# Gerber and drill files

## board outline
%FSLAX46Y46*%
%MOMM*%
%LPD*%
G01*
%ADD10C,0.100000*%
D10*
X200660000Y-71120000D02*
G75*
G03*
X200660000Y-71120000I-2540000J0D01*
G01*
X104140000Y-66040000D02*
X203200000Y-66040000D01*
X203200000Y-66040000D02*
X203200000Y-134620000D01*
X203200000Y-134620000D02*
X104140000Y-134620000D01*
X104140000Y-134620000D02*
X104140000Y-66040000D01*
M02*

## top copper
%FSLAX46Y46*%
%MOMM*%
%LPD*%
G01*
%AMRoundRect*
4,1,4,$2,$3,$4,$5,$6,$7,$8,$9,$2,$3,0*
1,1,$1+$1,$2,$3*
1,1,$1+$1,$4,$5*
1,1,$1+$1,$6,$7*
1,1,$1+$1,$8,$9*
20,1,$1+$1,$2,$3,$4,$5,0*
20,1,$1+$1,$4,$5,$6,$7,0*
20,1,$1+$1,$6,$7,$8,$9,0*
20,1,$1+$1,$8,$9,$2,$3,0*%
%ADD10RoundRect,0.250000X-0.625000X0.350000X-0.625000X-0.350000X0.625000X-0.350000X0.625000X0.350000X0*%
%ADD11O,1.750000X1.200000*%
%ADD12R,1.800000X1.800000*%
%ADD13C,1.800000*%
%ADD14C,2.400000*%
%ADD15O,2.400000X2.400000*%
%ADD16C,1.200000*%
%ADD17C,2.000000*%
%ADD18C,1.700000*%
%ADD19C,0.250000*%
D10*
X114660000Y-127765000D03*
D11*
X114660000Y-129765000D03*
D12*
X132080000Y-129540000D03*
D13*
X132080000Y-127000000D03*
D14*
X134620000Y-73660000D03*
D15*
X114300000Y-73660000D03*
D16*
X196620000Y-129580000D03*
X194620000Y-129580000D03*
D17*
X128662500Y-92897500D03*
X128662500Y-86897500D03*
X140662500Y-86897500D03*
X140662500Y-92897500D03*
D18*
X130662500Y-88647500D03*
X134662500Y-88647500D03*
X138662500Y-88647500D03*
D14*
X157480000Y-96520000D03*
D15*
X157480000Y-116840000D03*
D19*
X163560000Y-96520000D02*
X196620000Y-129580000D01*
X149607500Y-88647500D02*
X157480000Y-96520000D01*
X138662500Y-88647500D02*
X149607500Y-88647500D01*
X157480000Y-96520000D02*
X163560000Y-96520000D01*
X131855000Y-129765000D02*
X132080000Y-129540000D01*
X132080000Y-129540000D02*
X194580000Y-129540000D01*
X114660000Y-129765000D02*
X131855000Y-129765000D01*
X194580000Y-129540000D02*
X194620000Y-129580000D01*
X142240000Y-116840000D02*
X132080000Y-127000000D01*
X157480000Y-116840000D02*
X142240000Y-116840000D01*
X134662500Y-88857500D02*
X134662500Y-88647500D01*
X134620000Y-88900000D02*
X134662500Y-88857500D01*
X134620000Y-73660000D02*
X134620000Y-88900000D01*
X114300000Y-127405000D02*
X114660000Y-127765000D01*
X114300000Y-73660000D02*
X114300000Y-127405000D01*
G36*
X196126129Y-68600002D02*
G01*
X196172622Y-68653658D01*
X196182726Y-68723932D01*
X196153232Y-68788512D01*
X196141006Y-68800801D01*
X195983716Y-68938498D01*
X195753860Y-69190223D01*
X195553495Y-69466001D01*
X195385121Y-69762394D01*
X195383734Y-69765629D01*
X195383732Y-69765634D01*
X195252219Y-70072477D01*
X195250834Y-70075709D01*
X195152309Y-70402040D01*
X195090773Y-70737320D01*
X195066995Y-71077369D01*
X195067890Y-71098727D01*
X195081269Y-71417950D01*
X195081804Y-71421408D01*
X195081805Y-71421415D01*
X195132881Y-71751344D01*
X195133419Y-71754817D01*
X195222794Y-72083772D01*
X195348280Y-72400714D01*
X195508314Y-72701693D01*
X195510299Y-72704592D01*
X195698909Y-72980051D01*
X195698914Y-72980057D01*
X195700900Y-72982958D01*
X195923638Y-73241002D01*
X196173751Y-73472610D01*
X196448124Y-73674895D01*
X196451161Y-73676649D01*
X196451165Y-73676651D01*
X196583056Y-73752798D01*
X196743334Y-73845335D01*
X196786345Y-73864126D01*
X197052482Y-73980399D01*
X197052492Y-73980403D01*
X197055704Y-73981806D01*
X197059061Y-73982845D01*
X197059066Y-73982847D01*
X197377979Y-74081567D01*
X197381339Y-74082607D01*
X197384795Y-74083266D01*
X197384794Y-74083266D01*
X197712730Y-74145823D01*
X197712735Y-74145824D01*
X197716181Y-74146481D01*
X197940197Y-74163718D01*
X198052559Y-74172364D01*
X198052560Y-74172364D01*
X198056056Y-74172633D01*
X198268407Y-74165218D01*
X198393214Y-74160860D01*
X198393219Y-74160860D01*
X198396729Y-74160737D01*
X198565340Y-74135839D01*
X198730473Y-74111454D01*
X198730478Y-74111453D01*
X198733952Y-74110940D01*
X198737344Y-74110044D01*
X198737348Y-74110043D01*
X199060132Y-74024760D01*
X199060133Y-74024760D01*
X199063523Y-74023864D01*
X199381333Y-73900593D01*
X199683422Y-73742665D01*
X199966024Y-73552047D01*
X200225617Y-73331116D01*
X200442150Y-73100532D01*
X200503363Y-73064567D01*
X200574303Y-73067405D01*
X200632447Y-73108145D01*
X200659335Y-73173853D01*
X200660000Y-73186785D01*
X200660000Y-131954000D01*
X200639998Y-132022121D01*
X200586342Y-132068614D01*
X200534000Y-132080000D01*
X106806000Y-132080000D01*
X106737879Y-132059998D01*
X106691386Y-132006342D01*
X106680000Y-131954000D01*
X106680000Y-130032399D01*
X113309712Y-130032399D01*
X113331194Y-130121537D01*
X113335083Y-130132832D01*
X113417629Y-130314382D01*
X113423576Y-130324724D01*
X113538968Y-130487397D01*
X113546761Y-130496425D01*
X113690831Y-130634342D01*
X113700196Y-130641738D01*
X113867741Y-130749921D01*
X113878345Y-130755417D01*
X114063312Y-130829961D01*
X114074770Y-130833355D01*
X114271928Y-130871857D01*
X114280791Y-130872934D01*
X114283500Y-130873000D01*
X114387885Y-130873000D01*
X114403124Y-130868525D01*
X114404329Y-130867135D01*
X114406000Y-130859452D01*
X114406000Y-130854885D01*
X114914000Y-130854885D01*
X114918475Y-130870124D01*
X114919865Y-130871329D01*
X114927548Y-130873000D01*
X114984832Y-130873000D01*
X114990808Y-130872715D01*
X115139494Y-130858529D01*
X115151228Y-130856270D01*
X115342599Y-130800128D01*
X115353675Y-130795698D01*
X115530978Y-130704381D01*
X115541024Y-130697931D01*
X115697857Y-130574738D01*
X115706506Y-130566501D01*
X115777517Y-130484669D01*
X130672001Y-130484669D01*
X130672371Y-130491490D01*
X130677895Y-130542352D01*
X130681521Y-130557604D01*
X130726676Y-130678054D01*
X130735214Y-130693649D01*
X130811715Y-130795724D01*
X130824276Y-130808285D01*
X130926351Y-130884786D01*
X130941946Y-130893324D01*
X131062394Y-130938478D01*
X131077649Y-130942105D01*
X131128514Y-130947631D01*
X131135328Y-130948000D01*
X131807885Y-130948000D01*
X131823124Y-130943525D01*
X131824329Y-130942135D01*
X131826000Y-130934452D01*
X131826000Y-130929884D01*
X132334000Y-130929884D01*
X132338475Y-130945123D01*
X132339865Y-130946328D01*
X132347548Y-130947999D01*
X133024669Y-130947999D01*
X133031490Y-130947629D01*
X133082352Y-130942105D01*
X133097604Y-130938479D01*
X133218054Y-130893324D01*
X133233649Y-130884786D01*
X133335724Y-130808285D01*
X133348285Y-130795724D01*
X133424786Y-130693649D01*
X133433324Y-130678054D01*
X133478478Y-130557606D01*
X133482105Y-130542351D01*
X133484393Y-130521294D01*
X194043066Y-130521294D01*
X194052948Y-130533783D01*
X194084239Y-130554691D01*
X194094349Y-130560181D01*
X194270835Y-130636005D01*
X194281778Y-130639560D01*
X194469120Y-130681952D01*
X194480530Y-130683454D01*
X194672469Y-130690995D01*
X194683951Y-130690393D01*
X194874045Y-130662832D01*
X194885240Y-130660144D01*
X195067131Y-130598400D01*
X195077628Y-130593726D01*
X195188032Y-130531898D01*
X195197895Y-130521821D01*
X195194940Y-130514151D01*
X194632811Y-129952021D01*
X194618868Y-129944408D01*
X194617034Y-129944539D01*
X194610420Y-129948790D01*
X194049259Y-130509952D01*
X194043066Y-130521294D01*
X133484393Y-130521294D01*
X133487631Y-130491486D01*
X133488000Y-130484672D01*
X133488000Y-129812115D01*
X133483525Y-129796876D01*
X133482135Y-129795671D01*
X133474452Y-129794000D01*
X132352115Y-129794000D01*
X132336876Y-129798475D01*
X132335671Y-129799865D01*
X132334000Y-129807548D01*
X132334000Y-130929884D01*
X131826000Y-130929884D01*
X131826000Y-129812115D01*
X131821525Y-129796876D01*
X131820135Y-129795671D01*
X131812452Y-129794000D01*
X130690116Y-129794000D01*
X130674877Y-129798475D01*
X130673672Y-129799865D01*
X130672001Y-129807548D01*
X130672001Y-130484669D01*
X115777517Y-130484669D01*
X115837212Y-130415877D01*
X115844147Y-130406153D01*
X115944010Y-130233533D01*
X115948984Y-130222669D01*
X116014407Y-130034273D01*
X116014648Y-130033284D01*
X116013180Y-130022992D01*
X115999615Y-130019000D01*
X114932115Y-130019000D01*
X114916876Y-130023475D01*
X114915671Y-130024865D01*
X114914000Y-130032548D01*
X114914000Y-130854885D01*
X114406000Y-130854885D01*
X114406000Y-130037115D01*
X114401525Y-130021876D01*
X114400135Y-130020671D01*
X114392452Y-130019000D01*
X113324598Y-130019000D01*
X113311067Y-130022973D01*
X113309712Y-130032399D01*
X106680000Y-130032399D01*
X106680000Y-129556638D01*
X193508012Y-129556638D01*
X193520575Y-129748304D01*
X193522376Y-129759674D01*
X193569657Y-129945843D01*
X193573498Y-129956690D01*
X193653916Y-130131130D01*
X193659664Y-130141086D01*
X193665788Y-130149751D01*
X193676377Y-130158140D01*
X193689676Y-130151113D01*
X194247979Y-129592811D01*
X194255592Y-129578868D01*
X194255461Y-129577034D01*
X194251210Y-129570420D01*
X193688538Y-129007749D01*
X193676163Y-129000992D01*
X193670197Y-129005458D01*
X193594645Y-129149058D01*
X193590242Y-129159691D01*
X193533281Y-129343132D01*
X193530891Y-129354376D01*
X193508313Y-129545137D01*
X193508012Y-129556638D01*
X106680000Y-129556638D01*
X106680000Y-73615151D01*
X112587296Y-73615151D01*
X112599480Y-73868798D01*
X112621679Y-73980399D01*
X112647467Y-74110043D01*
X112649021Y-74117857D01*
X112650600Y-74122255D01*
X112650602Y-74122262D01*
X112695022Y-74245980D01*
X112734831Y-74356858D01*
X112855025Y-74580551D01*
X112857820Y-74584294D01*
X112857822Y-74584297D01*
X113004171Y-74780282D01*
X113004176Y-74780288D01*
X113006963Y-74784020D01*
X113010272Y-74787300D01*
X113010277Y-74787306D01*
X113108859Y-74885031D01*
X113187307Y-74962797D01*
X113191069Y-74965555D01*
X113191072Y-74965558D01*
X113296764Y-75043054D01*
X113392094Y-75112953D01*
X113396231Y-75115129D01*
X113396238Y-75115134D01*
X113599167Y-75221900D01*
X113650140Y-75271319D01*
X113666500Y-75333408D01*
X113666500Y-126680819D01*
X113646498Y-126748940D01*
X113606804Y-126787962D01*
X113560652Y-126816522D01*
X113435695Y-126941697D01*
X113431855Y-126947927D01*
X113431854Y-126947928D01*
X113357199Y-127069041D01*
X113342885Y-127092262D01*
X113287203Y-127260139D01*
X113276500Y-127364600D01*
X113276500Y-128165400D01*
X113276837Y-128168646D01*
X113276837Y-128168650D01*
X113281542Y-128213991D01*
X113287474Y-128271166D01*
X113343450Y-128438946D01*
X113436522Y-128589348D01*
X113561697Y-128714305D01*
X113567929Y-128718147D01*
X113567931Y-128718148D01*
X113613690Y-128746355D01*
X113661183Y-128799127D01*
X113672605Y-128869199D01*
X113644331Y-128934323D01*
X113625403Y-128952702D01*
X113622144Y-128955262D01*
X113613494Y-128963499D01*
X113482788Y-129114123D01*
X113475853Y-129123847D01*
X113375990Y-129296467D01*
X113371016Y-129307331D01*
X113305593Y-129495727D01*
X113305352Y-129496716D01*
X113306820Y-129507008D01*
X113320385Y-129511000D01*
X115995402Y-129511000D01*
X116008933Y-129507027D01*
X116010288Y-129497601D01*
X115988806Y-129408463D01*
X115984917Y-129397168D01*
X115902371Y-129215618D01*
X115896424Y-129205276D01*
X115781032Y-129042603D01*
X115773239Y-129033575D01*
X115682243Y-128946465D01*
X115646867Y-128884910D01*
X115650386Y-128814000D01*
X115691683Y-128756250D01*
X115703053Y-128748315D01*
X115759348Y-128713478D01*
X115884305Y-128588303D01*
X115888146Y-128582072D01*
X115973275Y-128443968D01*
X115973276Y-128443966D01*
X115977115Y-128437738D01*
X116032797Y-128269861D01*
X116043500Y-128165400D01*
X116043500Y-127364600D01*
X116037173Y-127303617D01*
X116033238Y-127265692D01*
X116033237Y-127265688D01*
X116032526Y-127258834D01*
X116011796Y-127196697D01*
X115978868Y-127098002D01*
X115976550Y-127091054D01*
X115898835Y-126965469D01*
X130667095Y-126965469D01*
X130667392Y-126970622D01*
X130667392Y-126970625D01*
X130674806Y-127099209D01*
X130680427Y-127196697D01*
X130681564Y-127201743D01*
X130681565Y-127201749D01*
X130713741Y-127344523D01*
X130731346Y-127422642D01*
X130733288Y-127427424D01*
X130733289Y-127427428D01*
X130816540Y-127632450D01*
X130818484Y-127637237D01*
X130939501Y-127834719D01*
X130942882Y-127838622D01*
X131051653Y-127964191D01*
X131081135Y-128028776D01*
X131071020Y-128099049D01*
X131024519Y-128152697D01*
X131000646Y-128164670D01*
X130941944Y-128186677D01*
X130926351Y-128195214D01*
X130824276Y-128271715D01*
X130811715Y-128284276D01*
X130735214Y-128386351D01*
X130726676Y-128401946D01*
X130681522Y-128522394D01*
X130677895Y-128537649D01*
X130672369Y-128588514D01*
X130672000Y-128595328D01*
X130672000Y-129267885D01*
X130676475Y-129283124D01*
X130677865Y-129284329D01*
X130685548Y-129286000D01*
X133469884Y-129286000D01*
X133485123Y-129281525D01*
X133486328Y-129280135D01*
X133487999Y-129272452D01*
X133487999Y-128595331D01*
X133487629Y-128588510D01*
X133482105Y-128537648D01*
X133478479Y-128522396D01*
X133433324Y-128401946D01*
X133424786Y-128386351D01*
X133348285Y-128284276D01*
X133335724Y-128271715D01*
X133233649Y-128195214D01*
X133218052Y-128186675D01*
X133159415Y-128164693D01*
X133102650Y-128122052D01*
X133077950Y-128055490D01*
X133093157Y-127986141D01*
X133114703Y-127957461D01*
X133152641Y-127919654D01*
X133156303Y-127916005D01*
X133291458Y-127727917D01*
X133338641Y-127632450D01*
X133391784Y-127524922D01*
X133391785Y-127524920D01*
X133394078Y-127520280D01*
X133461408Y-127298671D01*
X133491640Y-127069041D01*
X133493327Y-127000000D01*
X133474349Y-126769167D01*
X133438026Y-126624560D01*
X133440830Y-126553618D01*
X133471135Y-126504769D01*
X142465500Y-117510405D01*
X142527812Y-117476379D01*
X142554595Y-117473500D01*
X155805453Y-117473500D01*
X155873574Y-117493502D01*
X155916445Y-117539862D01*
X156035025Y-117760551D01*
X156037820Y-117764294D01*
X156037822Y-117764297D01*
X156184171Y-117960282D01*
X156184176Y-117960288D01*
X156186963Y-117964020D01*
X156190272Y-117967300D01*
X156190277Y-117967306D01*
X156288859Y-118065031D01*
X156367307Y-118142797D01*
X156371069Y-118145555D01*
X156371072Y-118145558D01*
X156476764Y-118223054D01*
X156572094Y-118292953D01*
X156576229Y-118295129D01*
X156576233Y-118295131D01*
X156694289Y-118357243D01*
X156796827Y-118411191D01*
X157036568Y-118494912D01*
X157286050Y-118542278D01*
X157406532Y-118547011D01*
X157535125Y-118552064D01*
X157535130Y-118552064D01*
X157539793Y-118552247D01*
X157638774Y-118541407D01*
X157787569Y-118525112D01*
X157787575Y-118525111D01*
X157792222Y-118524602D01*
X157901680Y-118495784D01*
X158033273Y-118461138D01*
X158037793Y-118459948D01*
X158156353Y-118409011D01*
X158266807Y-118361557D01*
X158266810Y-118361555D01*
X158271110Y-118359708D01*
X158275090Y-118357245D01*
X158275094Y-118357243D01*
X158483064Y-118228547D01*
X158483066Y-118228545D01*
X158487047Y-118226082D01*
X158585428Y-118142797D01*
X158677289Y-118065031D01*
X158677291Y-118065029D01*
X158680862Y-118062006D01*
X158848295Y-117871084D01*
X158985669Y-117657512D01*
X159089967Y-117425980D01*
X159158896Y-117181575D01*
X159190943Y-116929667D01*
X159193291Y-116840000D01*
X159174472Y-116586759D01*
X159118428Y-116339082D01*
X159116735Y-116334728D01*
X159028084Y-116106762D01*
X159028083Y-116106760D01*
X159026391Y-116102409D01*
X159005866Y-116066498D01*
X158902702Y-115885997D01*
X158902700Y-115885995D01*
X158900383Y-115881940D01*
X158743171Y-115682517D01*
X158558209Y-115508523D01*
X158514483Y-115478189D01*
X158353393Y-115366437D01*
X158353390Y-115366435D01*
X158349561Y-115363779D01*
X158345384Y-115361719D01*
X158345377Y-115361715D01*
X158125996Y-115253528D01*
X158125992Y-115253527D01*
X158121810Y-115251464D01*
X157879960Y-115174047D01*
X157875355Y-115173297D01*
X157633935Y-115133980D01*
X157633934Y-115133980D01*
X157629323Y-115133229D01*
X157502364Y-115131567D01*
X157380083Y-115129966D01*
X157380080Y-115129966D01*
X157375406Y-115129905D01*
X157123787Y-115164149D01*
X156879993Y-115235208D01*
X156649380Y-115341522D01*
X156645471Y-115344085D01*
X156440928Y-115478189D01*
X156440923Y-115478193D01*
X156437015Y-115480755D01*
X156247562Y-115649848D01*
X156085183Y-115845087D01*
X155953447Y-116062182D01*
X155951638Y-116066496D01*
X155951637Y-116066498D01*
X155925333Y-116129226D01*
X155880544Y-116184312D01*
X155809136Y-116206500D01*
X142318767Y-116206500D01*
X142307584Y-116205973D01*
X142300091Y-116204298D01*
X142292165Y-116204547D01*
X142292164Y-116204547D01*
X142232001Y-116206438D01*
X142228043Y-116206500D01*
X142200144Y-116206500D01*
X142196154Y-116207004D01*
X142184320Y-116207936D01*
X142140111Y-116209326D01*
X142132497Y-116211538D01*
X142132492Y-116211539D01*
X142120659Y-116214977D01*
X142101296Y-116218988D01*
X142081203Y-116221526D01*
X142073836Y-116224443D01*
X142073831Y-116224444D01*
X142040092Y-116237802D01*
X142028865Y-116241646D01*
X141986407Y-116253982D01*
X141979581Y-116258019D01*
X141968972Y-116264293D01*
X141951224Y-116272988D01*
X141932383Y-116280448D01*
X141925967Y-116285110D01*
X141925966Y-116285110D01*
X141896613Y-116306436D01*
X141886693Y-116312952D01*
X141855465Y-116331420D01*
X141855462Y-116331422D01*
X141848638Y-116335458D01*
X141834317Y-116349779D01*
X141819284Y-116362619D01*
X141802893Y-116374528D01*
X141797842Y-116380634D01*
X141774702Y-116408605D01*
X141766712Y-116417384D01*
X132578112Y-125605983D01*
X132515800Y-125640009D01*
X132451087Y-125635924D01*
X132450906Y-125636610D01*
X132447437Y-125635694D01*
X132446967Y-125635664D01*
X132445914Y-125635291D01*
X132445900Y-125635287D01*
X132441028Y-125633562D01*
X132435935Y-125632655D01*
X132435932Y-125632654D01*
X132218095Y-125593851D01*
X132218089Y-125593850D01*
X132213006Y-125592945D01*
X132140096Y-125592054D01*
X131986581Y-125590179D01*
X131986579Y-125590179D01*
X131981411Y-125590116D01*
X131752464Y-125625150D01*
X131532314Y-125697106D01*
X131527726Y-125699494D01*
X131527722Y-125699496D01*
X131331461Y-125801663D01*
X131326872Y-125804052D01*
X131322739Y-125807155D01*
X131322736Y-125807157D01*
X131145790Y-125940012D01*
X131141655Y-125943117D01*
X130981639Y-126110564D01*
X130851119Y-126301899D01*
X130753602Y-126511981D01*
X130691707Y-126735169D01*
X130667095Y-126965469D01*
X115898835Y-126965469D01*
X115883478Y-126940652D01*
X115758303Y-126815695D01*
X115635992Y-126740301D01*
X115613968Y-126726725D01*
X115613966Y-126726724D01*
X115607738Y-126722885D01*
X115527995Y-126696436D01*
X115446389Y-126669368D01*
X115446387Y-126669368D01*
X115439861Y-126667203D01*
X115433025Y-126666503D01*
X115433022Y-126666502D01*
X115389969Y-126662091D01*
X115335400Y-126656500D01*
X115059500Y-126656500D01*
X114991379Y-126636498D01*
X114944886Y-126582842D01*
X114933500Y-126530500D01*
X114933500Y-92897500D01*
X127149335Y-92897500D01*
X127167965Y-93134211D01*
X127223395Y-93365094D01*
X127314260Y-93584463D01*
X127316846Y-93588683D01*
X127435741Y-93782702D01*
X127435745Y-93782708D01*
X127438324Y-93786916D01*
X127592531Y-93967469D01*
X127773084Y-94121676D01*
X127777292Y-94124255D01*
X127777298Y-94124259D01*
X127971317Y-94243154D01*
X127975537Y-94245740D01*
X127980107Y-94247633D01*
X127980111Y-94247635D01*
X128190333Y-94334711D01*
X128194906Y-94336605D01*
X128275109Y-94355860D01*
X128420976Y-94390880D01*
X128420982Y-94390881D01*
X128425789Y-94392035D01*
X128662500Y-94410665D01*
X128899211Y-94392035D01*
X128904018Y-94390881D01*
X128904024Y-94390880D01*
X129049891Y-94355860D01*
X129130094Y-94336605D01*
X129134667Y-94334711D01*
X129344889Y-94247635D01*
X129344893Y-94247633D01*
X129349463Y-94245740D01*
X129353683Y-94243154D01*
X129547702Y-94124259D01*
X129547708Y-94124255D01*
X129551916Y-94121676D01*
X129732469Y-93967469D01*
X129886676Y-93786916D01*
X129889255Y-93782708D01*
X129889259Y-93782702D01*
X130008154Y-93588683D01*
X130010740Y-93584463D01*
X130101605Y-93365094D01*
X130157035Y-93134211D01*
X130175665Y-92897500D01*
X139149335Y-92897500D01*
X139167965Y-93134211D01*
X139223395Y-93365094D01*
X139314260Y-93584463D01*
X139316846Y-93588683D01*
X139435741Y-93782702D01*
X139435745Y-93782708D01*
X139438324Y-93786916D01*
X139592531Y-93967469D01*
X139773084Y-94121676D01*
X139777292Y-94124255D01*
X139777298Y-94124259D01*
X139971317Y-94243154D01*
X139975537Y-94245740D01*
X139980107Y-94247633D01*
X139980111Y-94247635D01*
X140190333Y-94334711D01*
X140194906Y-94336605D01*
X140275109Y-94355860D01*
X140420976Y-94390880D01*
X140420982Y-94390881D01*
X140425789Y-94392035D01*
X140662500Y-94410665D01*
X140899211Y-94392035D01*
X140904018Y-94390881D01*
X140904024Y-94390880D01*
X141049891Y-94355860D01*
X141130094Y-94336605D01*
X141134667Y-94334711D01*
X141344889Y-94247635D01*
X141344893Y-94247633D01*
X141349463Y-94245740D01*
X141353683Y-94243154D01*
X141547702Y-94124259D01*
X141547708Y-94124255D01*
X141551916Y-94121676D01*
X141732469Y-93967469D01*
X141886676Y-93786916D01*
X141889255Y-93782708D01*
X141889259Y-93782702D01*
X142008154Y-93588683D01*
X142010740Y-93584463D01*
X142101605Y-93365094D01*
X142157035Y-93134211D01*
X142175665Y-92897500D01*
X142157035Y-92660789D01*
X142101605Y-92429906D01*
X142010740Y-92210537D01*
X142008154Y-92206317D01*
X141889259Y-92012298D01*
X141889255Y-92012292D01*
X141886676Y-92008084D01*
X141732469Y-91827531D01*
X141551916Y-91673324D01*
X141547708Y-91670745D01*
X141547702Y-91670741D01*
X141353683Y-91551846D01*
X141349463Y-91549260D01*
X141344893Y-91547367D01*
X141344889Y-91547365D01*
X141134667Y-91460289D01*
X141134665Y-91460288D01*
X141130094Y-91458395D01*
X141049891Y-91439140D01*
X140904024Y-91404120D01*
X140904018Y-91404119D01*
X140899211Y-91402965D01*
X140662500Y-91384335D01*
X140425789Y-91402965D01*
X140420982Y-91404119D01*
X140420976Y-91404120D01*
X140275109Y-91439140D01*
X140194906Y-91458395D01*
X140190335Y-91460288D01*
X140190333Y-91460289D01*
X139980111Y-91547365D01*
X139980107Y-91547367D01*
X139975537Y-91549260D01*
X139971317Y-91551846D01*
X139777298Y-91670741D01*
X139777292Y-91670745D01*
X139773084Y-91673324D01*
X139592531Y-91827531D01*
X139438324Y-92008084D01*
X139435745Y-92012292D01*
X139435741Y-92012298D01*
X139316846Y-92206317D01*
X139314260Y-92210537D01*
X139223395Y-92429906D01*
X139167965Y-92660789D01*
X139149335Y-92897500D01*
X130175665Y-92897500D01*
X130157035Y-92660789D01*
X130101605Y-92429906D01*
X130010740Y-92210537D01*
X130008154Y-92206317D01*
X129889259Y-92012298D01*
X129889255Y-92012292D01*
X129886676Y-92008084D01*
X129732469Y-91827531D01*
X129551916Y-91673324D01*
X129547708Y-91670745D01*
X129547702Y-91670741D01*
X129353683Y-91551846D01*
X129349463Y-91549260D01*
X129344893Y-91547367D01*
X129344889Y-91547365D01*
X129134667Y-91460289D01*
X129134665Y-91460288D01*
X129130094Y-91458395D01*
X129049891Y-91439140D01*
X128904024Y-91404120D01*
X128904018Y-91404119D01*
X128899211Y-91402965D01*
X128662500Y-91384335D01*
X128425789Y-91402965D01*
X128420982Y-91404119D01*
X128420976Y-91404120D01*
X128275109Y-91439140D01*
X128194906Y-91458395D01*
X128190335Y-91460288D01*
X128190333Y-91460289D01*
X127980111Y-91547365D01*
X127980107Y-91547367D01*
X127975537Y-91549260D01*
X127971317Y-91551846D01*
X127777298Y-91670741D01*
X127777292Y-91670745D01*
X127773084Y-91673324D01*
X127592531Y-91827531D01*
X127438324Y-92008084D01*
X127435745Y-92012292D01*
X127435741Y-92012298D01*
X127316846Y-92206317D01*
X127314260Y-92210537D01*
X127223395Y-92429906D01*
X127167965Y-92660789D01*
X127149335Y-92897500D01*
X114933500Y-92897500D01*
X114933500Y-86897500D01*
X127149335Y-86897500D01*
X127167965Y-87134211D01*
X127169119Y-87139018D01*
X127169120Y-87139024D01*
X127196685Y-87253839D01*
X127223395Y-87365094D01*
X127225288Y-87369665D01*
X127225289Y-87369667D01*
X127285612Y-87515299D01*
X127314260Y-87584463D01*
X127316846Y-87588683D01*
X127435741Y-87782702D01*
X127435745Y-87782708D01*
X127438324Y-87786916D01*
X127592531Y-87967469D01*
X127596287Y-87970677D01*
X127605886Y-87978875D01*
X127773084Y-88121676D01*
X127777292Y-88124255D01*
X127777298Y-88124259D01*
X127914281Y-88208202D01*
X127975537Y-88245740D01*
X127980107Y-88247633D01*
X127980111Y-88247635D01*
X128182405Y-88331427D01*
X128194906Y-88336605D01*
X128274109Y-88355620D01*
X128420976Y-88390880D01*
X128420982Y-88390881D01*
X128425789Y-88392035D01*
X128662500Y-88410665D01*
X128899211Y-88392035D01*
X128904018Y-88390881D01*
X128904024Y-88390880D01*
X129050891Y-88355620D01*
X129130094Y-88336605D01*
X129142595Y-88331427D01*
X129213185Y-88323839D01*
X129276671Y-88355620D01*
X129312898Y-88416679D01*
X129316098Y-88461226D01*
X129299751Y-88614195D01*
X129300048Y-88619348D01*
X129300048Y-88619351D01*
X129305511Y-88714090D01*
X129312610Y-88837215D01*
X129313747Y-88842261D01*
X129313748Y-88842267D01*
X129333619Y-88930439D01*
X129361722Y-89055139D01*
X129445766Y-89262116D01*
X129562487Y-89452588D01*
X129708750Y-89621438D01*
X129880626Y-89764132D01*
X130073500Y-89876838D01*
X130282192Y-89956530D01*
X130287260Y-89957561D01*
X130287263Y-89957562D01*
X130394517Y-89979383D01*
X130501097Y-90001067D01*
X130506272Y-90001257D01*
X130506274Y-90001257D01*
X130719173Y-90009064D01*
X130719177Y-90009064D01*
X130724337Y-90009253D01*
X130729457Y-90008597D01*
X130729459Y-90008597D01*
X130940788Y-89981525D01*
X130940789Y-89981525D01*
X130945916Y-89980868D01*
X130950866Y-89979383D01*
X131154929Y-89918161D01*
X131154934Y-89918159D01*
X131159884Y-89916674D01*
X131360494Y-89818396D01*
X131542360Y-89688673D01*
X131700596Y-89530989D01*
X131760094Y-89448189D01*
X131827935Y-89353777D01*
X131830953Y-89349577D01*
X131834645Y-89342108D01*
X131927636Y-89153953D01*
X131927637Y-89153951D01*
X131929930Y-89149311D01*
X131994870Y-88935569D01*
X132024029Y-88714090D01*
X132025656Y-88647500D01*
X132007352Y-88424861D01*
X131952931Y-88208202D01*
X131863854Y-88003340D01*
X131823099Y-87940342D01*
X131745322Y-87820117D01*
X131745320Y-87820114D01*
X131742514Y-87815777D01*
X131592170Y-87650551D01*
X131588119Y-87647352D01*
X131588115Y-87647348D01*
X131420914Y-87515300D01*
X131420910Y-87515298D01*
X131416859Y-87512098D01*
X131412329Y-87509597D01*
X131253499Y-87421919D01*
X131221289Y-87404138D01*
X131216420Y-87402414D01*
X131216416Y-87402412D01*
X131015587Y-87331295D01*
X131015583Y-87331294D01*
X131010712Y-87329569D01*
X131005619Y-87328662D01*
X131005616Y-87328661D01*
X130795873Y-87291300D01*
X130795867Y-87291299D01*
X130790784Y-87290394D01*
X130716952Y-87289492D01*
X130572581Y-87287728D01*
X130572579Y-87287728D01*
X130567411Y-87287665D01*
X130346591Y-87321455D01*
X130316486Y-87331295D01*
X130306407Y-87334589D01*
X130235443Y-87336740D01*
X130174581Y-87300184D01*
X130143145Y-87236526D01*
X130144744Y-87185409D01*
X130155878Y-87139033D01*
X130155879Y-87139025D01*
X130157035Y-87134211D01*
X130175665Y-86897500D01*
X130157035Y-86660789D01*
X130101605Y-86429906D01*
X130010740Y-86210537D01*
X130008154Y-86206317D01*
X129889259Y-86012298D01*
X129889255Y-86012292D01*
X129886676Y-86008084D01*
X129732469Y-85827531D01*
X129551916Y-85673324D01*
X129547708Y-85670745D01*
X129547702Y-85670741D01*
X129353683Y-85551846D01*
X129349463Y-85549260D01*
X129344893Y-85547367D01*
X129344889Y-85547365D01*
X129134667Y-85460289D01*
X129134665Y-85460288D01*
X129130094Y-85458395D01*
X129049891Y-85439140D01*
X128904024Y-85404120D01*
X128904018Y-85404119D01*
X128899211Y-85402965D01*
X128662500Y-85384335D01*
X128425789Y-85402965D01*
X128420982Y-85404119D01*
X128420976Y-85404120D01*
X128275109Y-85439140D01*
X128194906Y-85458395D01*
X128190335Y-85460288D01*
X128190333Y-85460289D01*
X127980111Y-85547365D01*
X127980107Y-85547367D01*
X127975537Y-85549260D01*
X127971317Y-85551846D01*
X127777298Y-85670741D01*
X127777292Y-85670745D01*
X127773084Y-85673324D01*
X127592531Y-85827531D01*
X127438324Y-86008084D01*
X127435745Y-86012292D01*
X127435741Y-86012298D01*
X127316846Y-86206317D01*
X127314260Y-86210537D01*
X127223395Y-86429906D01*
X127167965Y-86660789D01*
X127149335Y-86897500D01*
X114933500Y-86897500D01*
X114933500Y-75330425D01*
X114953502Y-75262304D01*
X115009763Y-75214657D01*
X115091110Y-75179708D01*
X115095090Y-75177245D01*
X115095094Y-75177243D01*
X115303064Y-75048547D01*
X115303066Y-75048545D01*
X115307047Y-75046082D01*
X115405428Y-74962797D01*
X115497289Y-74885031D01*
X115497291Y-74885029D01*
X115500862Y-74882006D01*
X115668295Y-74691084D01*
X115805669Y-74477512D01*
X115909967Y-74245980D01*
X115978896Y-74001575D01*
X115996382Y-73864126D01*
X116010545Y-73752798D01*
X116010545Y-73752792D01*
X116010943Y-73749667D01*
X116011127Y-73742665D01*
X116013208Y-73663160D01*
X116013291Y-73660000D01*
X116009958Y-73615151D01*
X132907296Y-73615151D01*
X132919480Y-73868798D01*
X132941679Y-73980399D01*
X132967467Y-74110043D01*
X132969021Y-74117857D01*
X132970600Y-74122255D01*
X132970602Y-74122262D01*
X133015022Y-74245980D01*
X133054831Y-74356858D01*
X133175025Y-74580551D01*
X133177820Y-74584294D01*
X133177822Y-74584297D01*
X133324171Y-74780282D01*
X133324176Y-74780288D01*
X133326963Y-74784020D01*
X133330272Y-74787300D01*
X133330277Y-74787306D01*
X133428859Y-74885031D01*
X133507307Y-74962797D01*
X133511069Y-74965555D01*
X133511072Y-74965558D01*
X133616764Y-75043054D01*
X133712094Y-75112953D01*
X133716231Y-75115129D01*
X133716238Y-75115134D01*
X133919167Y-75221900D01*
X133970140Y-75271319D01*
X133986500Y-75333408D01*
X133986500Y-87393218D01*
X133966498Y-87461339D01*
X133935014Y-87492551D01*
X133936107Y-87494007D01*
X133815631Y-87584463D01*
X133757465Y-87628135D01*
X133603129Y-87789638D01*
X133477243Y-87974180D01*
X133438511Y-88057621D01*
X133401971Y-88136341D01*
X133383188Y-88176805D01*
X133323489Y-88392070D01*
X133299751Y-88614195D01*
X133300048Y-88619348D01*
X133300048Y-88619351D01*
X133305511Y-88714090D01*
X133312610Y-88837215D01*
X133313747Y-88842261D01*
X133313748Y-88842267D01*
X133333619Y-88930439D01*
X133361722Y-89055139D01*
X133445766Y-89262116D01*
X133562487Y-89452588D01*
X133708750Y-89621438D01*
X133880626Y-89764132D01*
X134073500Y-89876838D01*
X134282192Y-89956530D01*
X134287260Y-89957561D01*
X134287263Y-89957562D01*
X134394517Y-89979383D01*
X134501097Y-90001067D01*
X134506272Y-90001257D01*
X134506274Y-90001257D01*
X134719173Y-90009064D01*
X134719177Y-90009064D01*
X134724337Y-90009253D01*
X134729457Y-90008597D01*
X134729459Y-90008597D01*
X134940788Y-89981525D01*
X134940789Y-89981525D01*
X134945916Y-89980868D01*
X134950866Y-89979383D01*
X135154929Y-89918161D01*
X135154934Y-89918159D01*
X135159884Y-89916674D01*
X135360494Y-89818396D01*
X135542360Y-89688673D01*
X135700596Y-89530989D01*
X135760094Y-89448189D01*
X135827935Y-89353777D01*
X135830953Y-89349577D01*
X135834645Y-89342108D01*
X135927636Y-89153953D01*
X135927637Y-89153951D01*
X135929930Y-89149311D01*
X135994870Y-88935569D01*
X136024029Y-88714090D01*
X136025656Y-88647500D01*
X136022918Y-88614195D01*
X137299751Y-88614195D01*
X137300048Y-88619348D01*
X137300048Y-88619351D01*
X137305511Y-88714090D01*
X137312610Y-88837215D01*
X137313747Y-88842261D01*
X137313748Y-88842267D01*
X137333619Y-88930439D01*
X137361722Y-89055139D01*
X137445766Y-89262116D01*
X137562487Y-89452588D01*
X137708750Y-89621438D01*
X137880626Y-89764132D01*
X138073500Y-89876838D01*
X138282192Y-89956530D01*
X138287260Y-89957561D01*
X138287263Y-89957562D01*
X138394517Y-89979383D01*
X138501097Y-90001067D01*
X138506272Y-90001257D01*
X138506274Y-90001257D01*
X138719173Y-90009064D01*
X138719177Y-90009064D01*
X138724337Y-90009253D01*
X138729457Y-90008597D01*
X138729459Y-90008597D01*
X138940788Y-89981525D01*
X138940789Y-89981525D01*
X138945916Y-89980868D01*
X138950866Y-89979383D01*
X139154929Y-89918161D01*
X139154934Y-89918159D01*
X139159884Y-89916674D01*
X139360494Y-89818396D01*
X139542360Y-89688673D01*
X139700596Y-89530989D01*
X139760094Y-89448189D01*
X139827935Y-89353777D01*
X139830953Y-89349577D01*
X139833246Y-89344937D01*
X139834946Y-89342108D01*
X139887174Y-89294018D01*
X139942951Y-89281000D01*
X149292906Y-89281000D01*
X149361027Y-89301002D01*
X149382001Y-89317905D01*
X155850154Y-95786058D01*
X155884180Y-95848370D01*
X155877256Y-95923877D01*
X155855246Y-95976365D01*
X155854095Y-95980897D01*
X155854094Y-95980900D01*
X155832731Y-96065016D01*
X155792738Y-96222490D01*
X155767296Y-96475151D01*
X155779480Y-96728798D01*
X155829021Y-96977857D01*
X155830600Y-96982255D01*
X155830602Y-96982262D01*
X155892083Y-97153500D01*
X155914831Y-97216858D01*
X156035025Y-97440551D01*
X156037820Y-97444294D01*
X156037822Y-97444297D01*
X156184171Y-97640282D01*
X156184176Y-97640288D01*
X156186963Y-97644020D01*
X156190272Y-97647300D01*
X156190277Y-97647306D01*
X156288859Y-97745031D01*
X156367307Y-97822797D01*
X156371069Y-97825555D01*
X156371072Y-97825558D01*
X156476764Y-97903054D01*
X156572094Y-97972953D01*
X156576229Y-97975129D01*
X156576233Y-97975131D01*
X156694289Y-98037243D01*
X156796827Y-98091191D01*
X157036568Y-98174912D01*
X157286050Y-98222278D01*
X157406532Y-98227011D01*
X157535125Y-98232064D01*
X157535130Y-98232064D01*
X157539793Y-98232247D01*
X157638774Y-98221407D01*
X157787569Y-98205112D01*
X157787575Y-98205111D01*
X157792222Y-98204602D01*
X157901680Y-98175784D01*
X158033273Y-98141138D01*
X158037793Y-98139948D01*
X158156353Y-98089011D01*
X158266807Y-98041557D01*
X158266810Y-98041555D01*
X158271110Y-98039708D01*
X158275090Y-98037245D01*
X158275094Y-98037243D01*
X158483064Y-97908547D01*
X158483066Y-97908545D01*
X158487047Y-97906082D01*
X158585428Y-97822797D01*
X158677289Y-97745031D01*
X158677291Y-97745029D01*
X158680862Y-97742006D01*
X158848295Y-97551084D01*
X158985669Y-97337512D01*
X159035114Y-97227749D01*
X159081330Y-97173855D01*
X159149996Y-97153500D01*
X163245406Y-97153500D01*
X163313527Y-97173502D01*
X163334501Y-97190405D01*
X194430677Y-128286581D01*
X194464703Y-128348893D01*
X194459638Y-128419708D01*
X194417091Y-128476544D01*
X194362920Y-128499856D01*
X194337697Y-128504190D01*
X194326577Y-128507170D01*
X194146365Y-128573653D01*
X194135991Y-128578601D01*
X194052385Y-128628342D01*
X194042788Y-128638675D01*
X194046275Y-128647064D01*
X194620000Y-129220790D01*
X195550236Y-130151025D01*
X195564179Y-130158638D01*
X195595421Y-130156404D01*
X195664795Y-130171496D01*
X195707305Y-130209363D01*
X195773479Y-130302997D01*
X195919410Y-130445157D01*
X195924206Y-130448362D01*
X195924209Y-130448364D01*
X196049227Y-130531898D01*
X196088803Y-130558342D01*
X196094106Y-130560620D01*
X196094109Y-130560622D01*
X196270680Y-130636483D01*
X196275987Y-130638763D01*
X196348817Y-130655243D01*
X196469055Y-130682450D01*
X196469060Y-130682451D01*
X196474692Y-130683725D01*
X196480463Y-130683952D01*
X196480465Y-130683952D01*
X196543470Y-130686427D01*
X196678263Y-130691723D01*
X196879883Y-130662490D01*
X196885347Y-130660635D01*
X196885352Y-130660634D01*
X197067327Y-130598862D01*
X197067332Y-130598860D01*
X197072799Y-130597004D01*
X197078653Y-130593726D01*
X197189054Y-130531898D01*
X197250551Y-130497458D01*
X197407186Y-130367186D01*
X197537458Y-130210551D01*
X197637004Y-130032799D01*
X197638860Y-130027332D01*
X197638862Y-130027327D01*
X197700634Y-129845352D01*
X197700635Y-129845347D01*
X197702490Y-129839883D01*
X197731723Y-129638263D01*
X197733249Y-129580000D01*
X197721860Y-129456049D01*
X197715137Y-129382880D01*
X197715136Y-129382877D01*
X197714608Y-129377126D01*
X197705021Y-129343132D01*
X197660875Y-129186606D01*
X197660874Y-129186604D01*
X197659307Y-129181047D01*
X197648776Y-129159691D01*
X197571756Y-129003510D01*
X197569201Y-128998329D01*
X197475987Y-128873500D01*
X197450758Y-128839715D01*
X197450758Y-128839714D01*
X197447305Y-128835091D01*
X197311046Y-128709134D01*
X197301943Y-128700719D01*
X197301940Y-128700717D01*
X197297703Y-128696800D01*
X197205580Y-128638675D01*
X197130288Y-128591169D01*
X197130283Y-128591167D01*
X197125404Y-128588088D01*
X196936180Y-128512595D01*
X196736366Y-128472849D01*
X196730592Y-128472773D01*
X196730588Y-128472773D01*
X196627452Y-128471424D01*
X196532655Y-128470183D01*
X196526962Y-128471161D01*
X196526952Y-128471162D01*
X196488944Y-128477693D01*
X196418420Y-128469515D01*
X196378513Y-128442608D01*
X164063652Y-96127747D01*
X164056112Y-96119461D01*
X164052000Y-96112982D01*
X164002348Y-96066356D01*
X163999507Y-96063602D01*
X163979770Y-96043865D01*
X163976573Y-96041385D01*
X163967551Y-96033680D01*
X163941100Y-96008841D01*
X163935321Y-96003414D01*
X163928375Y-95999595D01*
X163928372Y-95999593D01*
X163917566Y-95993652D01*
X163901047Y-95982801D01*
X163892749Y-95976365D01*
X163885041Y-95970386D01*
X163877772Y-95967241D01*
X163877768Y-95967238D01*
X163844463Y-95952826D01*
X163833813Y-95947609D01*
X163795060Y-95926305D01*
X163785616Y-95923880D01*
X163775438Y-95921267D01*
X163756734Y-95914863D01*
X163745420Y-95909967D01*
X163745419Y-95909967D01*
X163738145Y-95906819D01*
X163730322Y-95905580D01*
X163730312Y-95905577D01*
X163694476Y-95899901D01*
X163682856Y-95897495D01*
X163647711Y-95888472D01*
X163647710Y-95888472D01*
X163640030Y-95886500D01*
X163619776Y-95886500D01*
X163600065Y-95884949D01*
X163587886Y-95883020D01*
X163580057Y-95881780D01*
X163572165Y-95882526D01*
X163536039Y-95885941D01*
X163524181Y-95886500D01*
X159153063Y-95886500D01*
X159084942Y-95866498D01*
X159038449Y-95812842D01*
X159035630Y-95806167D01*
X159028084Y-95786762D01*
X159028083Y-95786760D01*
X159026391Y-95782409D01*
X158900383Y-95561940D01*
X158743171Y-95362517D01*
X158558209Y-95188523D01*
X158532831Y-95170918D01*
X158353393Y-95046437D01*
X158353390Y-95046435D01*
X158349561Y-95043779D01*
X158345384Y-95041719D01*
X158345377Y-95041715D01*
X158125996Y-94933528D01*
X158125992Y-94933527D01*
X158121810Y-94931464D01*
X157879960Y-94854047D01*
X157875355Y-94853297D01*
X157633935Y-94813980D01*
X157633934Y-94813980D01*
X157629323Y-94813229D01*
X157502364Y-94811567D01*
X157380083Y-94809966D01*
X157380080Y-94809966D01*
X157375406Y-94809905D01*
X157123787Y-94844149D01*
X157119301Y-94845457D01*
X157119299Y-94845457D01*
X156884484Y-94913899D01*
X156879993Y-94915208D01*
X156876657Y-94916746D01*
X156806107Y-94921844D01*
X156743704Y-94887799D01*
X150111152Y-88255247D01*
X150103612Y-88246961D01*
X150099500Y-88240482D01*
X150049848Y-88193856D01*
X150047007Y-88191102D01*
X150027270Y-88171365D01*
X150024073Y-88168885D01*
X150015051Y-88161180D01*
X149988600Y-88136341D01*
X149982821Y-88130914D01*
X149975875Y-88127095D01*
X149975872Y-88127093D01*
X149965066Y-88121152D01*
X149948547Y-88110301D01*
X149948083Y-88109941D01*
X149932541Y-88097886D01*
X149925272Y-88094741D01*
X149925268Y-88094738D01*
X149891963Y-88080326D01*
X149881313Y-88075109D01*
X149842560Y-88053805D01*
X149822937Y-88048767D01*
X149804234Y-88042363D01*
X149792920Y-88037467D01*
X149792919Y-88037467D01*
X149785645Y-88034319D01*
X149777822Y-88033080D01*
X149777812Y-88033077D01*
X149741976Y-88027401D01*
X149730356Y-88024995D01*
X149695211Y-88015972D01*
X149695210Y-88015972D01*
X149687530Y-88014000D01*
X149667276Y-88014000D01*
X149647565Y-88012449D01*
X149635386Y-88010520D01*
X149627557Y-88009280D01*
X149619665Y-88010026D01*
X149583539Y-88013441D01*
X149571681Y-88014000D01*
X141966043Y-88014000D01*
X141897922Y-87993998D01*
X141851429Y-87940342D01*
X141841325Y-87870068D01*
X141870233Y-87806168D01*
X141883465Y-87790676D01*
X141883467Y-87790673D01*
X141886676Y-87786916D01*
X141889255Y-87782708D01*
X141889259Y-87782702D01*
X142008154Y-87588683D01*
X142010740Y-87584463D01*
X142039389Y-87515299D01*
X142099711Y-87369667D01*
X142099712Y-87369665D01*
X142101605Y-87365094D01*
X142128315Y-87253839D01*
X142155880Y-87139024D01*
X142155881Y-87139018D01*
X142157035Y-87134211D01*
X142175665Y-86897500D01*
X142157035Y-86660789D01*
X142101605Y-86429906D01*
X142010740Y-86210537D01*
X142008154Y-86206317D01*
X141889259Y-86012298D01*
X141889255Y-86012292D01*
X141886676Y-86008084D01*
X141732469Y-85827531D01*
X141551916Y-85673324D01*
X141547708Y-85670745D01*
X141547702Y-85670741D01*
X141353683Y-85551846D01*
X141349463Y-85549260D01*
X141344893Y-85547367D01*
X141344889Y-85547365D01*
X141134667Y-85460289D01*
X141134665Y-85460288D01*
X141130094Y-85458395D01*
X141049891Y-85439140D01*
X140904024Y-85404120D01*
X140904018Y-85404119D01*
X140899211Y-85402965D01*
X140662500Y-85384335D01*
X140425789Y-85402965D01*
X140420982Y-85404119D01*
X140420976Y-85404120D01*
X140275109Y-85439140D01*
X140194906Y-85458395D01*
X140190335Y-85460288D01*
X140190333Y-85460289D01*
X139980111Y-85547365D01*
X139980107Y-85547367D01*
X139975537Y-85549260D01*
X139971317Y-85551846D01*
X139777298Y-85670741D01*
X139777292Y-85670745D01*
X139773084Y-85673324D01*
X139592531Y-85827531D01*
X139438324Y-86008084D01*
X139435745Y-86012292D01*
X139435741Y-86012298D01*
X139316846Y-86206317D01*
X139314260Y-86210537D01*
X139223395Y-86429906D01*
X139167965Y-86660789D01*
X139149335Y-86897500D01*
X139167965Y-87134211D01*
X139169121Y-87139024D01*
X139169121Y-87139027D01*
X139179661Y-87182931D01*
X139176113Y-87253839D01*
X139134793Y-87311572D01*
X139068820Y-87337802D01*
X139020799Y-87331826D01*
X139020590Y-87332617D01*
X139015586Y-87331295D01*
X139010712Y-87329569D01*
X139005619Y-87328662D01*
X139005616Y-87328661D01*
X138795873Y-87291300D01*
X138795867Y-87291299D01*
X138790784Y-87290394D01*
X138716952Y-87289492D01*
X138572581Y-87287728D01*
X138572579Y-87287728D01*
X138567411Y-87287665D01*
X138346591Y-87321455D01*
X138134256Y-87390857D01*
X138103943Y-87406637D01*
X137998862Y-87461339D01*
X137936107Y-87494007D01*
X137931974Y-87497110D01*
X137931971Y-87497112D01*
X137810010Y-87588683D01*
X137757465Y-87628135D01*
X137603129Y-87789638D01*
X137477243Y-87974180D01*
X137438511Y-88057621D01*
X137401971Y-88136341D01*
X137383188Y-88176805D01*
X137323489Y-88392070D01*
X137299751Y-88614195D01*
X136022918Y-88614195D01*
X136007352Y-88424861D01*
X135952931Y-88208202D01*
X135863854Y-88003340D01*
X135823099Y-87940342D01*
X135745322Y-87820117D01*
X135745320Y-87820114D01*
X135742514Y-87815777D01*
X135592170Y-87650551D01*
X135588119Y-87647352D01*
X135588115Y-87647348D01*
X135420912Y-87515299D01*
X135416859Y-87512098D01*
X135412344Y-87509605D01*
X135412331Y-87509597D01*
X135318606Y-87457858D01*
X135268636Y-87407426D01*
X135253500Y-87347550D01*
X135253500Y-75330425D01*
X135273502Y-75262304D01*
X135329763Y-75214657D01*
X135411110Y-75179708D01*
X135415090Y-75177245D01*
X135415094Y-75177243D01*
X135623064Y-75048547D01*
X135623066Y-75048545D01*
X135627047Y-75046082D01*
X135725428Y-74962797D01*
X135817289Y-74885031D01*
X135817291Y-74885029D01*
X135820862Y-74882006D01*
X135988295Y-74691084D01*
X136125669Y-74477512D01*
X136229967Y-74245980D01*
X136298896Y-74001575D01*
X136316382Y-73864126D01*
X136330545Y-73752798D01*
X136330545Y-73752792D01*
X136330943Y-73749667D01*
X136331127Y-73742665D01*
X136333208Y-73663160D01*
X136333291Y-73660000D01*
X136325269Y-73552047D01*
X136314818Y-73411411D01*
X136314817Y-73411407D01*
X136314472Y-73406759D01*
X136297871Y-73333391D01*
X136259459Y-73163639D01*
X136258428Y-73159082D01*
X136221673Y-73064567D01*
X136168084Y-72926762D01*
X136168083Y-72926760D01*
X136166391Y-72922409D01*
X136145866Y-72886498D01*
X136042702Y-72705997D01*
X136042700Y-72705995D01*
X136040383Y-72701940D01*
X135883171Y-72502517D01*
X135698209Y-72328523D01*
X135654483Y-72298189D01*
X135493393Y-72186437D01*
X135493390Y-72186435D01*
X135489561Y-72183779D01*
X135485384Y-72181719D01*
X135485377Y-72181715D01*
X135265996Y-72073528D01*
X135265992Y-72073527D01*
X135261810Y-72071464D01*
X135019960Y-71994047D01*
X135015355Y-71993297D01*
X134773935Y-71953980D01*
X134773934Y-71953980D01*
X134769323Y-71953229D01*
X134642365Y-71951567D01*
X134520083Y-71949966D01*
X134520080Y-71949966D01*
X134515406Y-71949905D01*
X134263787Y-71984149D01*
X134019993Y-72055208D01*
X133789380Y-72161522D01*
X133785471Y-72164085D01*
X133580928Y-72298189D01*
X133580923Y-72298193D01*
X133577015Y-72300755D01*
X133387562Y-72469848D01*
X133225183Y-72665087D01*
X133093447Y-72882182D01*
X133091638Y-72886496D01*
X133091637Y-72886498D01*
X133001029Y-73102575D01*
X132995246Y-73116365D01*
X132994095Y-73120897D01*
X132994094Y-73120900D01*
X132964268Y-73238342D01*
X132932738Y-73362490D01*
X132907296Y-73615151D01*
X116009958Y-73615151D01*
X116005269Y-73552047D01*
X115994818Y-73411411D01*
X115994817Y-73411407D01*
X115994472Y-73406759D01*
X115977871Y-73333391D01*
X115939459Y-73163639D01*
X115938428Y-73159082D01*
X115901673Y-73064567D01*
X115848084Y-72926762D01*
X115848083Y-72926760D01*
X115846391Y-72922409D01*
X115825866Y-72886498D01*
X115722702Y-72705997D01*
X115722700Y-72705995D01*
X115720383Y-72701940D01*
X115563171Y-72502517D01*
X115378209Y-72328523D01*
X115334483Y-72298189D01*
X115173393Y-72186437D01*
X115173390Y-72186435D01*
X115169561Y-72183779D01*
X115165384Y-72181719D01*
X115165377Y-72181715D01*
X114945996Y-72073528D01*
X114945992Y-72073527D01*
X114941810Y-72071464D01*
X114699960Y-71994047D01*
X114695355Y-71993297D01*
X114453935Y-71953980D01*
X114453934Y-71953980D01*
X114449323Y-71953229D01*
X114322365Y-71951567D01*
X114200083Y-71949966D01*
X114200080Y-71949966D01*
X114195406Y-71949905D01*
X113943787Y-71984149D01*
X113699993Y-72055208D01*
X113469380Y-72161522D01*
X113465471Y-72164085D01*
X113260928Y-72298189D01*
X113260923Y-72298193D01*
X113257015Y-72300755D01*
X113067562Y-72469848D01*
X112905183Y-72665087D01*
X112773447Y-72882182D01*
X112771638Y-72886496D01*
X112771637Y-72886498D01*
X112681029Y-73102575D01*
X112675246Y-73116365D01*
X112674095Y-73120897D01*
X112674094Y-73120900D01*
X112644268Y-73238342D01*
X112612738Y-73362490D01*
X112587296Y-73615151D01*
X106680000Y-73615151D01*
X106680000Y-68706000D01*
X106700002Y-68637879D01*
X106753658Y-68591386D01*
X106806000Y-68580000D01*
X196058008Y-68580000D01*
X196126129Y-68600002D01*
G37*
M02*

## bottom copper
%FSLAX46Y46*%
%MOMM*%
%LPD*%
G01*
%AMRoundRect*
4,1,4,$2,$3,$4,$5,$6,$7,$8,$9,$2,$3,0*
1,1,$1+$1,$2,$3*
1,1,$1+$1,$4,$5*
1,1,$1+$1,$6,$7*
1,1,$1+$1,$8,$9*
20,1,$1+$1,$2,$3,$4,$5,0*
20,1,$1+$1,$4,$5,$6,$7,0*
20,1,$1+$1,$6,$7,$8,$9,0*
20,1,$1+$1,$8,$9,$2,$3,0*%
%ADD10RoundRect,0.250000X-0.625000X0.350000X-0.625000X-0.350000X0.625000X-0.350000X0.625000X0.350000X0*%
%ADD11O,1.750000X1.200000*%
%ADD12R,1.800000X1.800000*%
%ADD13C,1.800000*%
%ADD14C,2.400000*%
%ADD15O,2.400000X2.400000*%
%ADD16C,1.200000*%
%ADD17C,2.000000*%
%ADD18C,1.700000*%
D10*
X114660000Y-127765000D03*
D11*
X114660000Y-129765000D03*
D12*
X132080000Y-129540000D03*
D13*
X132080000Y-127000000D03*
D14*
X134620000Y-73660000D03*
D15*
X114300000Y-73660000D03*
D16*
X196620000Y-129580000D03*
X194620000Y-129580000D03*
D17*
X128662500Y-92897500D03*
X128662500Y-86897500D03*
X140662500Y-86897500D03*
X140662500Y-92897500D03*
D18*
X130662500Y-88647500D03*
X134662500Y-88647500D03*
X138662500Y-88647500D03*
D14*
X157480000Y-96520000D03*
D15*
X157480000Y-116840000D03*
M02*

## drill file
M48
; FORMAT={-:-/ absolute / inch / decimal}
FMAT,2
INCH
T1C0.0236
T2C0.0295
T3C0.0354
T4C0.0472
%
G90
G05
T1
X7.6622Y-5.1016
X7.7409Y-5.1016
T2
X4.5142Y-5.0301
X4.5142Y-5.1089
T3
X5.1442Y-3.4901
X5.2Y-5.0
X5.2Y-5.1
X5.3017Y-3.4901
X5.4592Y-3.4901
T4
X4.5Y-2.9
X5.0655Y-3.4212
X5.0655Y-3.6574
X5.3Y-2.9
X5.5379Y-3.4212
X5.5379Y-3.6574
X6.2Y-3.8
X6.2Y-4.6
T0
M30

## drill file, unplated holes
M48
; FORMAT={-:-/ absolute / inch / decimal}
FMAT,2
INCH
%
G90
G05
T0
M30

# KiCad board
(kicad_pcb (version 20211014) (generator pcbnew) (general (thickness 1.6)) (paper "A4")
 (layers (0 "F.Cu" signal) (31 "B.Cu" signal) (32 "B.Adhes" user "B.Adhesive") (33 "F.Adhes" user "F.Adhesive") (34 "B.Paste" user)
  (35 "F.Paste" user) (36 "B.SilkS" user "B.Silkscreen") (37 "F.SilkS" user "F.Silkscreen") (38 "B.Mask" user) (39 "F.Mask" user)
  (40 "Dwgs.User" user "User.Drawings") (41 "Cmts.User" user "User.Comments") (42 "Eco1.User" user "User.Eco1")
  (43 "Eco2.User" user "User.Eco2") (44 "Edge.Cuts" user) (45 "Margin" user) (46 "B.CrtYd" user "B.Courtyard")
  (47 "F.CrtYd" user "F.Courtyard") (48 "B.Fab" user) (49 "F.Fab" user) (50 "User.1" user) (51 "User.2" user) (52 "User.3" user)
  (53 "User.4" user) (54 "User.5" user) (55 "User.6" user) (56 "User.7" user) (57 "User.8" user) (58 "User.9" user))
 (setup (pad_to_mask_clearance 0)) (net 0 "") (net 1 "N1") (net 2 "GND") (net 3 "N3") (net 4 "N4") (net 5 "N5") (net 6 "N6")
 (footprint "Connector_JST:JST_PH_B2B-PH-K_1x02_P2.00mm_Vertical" (layer "F.Cu") (at 114.66 127.765 -90)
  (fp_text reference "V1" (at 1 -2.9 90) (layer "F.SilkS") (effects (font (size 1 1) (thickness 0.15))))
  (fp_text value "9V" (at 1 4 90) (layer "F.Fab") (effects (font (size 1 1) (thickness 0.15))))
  (pad "1" thru_hole roundrect (at 0 0 270) (size 1.2 1.75) (drill 0.75) (layers *.Cu *.Mask) (roundrect_rratio 0.2083333333) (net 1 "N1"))
  (pad "2" thru_hole oval (at 2 0 270) (size 1.2 1.75) (drill 0.75) (layers *.Cu *.Mask) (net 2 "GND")))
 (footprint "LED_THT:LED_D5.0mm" (layer "F.Cu") (at 132.08 129.54 90)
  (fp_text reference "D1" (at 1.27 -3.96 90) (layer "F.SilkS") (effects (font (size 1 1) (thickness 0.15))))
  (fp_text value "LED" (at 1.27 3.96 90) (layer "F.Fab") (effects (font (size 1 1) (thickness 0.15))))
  (pad "1" thru_hole rect (at 0 0 90) (size 1.8 1.8) (drill 0.9) (layers *.Cu *.Mask) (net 2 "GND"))
  (pad "2" thru_hole circle (at 2.54 0 90) (size 1.8 1.8) (drill 0.9) (layers *.Cu *.Mask) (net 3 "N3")))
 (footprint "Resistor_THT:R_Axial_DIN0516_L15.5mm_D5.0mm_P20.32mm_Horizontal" (layer "F.Cu") (at 134.62 73.66 180)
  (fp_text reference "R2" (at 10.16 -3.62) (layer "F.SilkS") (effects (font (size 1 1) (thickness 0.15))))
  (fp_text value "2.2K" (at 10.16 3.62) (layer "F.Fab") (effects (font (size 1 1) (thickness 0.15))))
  (pad "1" thru_hole circle (at 0 0 180) (size 2.4 2.4) (drill 1.2) (layers *.Cu *.Mask) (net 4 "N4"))
  (pad "2" thru_hole oval (at 20.32 0 180) (size 2.4 2.4) (drill 1.2) (layers *.Cu *.Mask) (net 1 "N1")))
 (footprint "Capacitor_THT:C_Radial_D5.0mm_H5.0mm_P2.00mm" (layer "F.Cu") (at 196.62 129.58 180)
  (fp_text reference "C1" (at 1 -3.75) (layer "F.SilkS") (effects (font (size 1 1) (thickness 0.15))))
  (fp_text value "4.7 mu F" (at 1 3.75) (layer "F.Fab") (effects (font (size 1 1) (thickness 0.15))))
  (pad "1" thru_hole circle (at 0 0 180) (size 1.2 1.2) (drill 0.6) (layers *.Cu *.Mask) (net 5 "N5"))
  (pad "2" thru_hole circle (at 2 0 180) (size 1.2 1.2) (drill 0.6) (layers *.Cu *.Mask) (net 2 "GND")))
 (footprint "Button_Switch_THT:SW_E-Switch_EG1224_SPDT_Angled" (layer "F.Cu") (at 130.6625 88.6475)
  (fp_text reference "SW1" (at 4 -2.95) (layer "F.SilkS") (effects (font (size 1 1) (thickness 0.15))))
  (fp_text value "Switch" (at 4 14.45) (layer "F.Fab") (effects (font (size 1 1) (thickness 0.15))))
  (pad "" thru_hole circle (at -2 4.25) (size 2 2) (drill 1.2) (layers *.Cu *.Mask))
  (pad "" thru_hole circle (at -2 -1.75) (size 2 2) (drill 1.2) (layers *.Cu *.Mask))
  (pad "" thru_hole circle (at 10 -1.75) (size 2 2) (drill 1.2) (layers *.Cu *.Mask))
  (pad "" thru_hole circle (at 10 4.25) (size 2 2) (drill 1.2) (layers *.Cu *.Mask))
  (pad "1" thru_hole circle (at 0 0) (size 1.7 1.7) (drill 0.9) (layers *.Cu *.Mask) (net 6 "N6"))
  (pad "2" thru_hole circle (at 4 0) (size 1.7 1.7) (drill 0.9) (layers *.Cu *.Mask) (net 4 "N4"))
  (pad "3" thru_hole circle (at 8 0) (size 1.7 1.7) (drill 0.9) (layers *.Cu *.Mask) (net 5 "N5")))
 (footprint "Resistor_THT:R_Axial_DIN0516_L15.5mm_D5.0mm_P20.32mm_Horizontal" (layer "F.Cu") (at 157.48 96.52 -90)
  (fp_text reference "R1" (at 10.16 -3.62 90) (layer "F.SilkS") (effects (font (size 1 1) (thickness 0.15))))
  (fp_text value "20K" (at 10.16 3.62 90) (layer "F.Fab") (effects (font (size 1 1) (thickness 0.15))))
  (pad "1" thru_hole circle (at 0 0 270) (size 2.4 2.4) (drill 1.2) (layers *.Cu *.Mask) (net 5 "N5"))
  (pad "2" thru_hole oval (at 20.32 0 270) (size 2.4 2.4) (drill 1.2) (layers *.Cu *.Mask) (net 3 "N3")))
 (gr_circle (center 198.12 71.12) (end 198.12 73.66) (layer "Edge.Cuts") (width 0.1) (fill none))
 (gr_rect (start 104.14 66.04) (end 203.2 134.62) (layer "Edge.Cuts") (width 0.1) (fill none))
 (segment (start 163.56 96.52) (end 196.62 129.58) (width 0.25) (layer "F.Cu") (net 5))
 (segment (start 149.6075 88.6475) (end 157.48 96.52) (width 0.25) (layer "F.Cu") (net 5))
 (segment (start 138.6625 88.6475) (end 149.6075 88.6475) (width 0.25) (layer "F.Cu") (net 5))
 (segment (start 157.48 96.52) (end 163.56 96.52) (width 0.25) (layer "F.Cu") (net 5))
 (segment (start 131.855 129.765) (end 132.08 129.54) (width 0.25) (layer "F.Cu") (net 2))
 (segment (start 132.08 129.54) (end 194.58 129.54) (width 0.25) (layer "F.Cu") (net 2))
 (segment (start 114.66 129.765) (end 131.855 129.765) (width 0.25) (layer "F.Cu") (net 2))
 (segment (start 194.58 129.54) (end 194.62 129.58) (width 0.25) (layer "F.Cu") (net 2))
 (segment (start 142.24 116.84) (end 132.08 127) (width 0.25) (layer "F.Cu") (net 3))
 (segment (start 157.48 116.84) (end 142.24 116.84) (width 0.25) (layer "F.Cu") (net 3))
 (segment (start 134.6625 88.8575) (end 134.6625 88.6475) (width 0.25) (layer "F.Cu") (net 4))
 (segment (start 134.62 88.9) (end 134.6625 88.8575) (width 0.25) (layer "F.Cu") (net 4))
 (segment (start 134.62 73.66) (end 134.62 88.9) (width 0.25) (layer "F.Cu") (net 4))
 (segment (start 114.3 127.405) (end 114.66 127.765) (width 0.25) (layer "F.Cu") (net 1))
 (segment (start 114.3 73.66) (end 114.3 127.405) (width 0.25) (layer "F.Cu") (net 1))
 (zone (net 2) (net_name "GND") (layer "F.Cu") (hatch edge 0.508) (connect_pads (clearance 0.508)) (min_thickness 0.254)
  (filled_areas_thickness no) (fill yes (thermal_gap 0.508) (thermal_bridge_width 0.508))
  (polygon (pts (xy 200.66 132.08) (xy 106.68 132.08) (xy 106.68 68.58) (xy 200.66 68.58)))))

